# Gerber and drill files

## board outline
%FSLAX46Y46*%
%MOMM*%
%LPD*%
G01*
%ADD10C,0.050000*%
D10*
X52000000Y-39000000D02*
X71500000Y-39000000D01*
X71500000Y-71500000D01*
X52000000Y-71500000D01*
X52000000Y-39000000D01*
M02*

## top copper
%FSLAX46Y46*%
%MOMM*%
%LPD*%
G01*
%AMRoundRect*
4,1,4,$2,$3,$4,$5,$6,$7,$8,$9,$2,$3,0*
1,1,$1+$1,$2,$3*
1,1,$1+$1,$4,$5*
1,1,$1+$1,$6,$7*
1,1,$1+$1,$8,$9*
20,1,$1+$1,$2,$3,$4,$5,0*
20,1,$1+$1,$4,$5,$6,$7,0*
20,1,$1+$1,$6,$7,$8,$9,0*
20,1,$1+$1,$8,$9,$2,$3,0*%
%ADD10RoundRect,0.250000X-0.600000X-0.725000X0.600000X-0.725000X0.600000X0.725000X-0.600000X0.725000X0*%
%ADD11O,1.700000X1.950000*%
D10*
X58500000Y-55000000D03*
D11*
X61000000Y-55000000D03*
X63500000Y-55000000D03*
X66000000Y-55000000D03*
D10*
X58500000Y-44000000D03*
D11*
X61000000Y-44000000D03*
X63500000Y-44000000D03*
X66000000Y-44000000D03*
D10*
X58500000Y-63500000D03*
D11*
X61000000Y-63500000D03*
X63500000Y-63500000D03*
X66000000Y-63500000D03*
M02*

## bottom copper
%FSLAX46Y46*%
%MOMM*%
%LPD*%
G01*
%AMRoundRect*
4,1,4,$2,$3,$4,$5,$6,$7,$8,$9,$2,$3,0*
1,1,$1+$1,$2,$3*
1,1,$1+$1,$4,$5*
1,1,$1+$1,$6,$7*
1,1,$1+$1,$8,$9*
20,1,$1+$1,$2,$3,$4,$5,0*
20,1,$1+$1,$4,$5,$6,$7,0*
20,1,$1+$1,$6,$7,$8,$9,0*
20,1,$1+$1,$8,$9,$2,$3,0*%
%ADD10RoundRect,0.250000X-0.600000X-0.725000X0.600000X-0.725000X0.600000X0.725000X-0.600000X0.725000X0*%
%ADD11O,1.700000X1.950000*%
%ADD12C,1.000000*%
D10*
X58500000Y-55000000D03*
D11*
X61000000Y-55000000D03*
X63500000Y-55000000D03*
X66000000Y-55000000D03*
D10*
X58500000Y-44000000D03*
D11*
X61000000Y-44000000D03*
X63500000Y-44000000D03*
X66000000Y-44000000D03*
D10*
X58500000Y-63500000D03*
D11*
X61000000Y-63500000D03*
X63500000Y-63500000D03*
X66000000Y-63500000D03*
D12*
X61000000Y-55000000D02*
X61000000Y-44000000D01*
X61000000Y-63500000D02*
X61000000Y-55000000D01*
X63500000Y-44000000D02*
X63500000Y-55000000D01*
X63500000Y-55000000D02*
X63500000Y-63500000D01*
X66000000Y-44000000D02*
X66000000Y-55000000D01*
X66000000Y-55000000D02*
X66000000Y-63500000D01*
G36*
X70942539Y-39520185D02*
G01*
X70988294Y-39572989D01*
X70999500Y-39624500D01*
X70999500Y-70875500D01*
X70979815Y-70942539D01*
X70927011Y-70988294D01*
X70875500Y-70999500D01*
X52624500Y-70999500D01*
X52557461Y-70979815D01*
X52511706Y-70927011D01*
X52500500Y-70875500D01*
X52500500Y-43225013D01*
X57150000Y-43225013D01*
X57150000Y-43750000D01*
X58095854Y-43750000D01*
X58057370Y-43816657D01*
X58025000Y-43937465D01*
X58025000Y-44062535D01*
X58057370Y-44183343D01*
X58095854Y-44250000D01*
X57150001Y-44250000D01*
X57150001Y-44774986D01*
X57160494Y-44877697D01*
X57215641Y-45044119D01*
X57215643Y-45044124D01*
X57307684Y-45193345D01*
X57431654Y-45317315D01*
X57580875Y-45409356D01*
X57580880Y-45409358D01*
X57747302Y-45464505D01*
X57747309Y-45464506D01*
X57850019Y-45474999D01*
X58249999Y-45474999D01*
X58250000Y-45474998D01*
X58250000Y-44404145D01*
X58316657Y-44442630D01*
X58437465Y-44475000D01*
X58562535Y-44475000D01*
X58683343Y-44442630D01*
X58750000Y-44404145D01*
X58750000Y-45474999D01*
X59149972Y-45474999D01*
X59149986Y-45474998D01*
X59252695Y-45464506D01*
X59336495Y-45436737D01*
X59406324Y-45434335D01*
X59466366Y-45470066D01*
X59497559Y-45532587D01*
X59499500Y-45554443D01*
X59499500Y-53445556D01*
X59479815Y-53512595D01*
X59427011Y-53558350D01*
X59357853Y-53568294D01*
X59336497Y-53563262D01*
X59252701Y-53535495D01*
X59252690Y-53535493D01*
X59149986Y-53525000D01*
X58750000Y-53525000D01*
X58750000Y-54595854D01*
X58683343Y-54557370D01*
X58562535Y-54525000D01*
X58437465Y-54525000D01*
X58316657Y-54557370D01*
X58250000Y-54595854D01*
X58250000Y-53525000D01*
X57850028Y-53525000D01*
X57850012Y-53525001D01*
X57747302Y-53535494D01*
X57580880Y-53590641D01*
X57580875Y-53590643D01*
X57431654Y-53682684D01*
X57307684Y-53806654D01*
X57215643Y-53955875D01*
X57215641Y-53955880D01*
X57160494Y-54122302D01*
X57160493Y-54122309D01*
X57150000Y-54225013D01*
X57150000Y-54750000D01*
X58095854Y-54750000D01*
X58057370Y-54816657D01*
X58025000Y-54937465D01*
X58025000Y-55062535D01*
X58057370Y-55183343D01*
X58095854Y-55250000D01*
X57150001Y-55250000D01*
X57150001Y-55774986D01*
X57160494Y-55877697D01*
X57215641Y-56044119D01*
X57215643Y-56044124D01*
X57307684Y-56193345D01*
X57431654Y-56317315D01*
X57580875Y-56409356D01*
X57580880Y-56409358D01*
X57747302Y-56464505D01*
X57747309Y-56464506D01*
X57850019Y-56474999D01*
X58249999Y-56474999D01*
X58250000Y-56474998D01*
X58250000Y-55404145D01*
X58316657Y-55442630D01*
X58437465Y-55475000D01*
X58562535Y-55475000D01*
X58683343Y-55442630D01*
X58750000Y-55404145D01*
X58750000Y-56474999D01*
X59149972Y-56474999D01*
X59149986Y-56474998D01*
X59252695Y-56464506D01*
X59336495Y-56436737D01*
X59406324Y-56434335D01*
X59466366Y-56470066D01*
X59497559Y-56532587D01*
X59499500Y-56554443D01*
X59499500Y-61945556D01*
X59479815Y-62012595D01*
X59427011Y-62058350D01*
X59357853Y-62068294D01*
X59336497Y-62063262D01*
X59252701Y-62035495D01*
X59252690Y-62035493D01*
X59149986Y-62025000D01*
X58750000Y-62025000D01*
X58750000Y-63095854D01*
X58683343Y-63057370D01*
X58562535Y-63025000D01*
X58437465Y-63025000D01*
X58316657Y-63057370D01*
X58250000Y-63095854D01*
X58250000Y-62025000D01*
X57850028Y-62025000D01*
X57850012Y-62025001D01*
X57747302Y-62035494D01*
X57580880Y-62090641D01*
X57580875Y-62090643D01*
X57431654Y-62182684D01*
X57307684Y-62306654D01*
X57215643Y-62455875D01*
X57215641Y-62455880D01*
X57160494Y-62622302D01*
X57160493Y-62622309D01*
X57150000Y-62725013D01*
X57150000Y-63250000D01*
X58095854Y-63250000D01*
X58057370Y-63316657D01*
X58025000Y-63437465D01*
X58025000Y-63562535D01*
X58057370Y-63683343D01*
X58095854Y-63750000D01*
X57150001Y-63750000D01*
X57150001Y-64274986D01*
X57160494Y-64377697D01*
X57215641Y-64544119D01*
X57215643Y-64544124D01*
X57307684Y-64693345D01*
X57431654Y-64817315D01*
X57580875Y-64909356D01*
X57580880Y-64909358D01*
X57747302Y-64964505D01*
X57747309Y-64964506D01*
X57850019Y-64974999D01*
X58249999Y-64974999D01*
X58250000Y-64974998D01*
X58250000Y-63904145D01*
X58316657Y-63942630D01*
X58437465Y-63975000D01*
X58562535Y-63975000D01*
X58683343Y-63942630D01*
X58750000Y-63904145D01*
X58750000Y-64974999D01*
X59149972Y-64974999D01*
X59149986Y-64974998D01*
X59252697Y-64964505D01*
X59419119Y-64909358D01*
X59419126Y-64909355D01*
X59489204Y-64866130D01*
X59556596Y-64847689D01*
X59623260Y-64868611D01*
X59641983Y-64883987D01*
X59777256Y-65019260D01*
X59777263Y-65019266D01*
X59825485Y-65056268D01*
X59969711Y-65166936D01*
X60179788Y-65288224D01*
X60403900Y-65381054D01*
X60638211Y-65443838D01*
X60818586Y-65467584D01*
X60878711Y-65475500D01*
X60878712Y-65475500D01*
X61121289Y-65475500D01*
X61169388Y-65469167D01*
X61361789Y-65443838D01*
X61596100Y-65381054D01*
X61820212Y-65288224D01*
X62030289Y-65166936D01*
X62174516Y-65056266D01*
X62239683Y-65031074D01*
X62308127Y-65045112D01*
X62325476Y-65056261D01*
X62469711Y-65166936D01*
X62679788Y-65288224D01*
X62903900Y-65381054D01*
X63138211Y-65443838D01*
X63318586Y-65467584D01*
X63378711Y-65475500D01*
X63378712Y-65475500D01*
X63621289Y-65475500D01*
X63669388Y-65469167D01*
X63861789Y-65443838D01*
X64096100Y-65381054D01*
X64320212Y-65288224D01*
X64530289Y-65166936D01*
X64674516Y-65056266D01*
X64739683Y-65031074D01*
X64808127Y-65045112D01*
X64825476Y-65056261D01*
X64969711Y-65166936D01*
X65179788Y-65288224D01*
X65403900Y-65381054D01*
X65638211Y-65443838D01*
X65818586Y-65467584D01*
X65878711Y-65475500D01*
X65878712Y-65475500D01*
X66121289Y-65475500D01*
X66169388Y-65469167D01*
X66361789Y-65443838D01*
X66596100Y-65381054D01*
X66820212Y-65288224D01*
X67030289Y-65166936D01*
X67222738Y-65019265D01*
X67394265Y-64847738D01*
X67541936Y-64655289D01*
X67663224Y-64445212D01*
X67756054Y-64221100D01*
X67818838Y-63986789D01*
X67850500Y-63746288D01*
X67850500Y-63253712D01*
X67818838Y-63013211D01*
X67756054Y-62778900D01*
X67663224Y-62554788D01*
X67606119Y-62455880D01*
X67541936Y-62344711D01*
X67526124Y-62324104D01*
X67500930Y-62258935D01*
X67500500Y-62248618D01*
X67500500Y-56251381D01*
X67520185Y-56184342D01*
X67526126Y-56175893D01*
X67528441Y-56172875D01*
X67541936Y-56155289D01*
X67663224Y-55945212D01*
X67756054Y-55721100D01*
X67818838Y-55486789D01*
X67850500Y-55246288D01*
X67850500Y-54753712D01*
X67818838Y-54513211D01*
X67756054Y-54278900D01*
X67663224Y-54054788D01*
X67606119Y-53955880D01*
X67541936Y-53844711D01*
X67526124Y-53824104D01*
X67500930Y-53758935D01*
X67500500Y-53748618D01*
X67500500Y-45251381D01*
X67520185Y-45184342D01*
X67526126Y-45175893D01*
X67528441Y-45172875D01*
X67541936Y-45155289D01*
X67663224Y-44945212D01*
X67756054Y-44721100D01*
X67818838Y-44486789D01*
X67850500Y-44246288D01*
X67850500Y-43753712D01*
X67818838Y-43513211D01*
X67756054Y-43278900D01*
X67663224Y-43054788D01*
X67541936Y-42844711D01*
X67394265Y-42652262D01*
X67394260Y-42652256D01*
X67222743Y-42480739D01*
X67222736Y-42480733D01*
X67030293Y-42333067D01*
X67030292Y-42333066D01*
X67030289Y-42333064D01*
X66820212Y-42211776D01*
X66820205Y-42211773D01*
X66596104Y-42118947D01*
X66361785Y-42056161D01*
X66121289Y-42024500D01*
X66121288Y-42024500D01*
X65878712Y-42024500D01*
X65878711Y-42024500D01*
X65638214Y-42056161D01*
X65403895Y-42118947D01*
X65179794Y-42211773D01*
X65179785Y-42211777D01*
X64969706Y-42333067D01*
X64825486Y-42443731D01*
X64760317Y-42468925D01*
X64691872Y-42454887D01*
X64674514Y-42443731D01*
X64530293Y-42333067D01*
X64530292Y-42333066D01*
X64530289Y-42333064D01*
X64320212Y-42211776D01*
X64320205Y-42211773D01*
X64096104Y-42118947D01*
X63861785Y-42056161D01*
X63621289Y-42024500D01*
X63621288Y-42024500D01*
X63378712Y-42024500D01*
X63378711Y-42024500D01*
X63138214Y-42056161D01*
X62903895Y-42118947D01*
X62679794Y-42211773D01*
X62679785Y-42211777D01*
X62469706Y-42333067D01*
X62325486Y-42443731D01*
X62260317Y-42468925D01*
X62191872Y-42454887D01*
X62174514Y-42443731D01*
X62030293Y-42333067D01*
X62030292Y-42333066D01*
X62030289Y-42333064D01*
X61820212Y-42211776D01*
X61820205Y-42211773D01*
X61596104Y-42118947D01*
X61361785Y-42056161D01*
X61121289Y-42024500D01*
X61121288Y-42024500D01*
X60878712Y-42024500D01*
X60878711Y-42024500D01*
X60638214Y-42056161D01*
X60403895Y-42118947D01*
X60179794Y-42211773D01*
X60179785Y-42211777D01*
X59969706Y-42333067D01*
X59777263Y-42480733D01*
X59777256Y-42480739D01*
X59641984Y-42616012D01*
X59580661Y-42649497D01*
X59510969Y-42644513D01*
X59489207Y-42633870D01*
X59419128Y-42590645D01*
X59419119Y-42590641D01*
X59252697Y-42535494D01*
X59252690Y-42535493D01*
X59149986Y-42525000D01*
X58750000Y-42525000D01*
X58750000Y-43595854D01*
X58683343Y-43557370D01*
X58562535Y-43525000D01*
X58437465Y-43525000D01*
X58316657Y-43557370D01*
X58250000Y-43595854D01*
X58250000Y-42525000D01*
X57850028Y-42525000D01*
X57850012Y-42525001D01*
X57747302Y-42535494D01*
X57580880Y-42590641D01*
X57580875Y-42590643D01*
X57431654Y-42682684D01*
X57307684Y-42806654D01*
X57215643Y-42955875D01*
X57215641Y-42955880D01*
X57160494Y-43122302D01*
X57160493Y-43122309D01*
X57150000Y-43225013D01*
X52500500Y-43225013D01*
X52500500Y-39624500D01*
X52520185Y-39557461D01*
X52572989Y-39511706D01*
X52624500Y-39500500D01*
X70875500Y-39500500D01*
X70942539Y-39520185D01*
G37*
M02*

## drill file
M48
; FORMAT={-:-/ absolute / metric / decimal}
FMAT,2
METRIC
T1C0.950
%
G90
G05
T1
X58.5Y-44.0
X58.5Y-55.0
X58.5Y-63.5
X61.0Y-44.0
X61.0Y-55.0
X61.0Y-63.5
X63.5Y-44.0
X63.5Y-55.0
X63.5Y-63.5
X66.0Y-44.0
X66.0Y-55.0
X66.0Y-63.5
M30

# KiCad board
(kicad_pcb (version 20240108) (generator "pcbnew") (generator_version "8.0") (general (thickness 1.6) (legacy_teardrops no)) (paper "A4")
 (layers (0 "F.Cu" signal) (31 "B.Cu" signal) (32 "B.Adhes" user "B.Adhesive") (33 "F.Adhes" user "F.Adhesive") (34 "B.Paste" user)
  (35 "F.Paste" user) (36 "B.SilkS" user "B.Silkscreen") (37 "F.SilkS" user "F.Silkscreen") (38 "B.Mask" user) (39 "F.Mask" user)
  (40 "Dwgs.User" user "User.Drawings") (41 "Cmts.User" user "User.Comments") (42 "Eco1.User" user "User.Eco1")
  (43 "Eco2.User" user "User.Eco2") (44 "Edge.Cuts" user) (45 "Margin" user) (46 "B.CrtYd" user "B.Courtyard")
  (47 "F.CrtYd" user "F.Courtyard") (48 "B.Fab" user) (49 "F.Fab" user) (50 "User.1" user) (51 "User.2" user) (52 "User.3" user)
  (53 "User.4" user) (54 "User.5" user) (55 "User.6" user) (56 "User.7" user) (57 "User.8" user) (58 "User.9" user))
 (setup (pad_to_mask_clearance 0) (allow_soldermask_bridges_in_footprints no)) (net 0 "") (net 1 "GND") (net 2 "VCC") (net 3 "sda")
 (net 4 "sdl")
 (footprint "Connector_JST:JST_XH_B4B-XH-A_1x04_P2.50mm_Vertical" (layer "F.Cu") (at 58.5 55)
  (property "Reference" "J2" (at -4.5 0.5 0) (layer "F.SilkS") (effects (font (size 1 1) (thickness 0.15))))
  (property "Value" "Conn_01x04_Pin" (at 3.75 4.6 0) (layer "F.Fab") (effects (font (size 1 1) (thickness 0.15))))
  (pad "1" thru_hole roundrect (at 0 0) (size 1.7 1.95) (drill 0.95) (layers "*.Cu" "*.Mask") (remove_unused_layers no)
   (roundrect_rratio 0.147059) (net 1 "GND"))
  (pad "2" thru_hole oval (at 2.5 0) (size 1.7 1.95) (drill 0.95) (layers "*.Cu" "*.Mask") (remove_unused_layers no) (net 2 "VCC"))
  (pad "3" thru_hole oval (at 5 0) (size 1.7 1.95) (drill 0.95) (layers "*.Cu" "*.Mask") (remove_unused_layers no) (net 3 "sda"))
  (pad "4" thru_hole oval (at 7.5 0) (size 1.7 1.95) (drill 0.95) (layers "*.Cu" "*.Mask") (remove_unused_layers no) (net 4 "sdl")))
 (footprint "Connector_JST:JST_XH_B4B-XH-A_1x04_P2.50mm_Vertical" (layer "F.Cu") (at 58.5 44)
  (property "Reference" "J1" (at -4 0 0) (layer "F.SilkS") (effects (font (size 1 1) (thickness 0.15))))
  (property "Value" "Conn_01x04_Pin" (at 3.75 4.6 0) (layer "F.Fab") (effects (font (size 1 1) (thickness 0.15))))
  (pad "1" thru_hole roundrect (at 0 0) (size 1.7 1.95) (drill 0.95) (layers "*.Cu" "*.Mask") (remove_unused_layers no)
   (roundrect_rratio 0.147059) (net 1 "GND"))
  (pad "2" thru_hole oval (at 2.5 0) (size 1.7 1.95) (drill 0.95) (layers "*.Cu" "*.Mask") (remove_unused_layers no) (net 2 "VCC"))
  (pad "3" thru_hole oval (at 5 0) (size 1.7 1.95) (drill 0.95) (layers "*.Cu" "*.Mask") (remove_unused_layers no) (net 3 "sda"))
  (pad "4" thru_hole oval (at 7.5 0) (size 1.7 1.95) (drill 0.95) (layers "*.Cu" "*.Mask") (remove_unused_layers no) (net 4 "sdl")))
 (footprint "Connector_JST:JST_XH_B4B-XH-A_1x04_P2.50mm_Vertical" (layer "F.Cu") (at 58.5 63.5)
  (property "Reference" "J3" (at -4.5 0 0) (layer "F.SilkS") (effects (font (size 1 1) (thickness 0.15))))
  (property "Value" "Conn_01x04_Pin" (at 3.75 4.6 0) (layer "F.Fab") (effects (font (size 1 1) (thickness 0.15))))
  (pad "1" thru_hole roundrect (at 0 0) (size 1.7 1.95) (drill 0.95) (layers "*.Cu" "*.Mask") (remove_unused_layers no)
   (roundrect_rratio 0.147059) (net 1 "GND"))
  (pad "2" thru_hole oval (at 2.5 0) (size 1.7 1.95) (drill 0.95) (layers "*.Cu" "*.Mask") (remove_unused_layers no) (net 2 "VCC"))
  (pad "3" thru_hole oval (at 5 0) (size 1.7 1.95) (drill 0.95) (layers "*.Cu" "*.Mask") (remove_unused_layers no) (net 3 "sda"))
  (pad "4" thru_hole oval (at 7.5 0) (size 1.7 1.95) (drill 0.95) (layers "*.Cu" "*.Mask") (remove_unused_layers no) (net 4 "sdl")))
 (gr_rect (start 52 39) (end 71.5 71.5) (stroke (width 0.05) (type default)) (fill none) (layer "Edge.Cuts"))
 (segment (start 61 55) (end 61 44) (width 1) (layer "B.Cu") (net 2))
 (segment (start 61 63.5) (end 61 55) (width 1) (layer "B.Cu") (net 2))
 (segment (start 63.5 44) (end 63.5 55) (width 1) (layer "B.Cu") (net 3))
 (segment (start 63.5 55) (end 63.5 63.5) (width 1) (layer "B.Cu") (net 3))
 (segment (start 66 44) (end 66 55) (width 1) (layer "B.Cu") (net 4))
 (segment (start 66 55) (end 66 63.5) (width 1) (layer "B.Cu") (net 4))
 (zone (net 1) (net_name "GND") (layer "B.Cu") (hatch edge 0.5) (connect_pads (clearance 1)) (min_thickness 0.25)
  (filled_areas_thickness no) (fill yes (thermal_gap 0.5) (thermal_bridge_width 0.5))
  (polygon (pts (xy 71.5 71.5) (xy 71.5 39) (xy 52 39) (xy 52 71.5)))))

